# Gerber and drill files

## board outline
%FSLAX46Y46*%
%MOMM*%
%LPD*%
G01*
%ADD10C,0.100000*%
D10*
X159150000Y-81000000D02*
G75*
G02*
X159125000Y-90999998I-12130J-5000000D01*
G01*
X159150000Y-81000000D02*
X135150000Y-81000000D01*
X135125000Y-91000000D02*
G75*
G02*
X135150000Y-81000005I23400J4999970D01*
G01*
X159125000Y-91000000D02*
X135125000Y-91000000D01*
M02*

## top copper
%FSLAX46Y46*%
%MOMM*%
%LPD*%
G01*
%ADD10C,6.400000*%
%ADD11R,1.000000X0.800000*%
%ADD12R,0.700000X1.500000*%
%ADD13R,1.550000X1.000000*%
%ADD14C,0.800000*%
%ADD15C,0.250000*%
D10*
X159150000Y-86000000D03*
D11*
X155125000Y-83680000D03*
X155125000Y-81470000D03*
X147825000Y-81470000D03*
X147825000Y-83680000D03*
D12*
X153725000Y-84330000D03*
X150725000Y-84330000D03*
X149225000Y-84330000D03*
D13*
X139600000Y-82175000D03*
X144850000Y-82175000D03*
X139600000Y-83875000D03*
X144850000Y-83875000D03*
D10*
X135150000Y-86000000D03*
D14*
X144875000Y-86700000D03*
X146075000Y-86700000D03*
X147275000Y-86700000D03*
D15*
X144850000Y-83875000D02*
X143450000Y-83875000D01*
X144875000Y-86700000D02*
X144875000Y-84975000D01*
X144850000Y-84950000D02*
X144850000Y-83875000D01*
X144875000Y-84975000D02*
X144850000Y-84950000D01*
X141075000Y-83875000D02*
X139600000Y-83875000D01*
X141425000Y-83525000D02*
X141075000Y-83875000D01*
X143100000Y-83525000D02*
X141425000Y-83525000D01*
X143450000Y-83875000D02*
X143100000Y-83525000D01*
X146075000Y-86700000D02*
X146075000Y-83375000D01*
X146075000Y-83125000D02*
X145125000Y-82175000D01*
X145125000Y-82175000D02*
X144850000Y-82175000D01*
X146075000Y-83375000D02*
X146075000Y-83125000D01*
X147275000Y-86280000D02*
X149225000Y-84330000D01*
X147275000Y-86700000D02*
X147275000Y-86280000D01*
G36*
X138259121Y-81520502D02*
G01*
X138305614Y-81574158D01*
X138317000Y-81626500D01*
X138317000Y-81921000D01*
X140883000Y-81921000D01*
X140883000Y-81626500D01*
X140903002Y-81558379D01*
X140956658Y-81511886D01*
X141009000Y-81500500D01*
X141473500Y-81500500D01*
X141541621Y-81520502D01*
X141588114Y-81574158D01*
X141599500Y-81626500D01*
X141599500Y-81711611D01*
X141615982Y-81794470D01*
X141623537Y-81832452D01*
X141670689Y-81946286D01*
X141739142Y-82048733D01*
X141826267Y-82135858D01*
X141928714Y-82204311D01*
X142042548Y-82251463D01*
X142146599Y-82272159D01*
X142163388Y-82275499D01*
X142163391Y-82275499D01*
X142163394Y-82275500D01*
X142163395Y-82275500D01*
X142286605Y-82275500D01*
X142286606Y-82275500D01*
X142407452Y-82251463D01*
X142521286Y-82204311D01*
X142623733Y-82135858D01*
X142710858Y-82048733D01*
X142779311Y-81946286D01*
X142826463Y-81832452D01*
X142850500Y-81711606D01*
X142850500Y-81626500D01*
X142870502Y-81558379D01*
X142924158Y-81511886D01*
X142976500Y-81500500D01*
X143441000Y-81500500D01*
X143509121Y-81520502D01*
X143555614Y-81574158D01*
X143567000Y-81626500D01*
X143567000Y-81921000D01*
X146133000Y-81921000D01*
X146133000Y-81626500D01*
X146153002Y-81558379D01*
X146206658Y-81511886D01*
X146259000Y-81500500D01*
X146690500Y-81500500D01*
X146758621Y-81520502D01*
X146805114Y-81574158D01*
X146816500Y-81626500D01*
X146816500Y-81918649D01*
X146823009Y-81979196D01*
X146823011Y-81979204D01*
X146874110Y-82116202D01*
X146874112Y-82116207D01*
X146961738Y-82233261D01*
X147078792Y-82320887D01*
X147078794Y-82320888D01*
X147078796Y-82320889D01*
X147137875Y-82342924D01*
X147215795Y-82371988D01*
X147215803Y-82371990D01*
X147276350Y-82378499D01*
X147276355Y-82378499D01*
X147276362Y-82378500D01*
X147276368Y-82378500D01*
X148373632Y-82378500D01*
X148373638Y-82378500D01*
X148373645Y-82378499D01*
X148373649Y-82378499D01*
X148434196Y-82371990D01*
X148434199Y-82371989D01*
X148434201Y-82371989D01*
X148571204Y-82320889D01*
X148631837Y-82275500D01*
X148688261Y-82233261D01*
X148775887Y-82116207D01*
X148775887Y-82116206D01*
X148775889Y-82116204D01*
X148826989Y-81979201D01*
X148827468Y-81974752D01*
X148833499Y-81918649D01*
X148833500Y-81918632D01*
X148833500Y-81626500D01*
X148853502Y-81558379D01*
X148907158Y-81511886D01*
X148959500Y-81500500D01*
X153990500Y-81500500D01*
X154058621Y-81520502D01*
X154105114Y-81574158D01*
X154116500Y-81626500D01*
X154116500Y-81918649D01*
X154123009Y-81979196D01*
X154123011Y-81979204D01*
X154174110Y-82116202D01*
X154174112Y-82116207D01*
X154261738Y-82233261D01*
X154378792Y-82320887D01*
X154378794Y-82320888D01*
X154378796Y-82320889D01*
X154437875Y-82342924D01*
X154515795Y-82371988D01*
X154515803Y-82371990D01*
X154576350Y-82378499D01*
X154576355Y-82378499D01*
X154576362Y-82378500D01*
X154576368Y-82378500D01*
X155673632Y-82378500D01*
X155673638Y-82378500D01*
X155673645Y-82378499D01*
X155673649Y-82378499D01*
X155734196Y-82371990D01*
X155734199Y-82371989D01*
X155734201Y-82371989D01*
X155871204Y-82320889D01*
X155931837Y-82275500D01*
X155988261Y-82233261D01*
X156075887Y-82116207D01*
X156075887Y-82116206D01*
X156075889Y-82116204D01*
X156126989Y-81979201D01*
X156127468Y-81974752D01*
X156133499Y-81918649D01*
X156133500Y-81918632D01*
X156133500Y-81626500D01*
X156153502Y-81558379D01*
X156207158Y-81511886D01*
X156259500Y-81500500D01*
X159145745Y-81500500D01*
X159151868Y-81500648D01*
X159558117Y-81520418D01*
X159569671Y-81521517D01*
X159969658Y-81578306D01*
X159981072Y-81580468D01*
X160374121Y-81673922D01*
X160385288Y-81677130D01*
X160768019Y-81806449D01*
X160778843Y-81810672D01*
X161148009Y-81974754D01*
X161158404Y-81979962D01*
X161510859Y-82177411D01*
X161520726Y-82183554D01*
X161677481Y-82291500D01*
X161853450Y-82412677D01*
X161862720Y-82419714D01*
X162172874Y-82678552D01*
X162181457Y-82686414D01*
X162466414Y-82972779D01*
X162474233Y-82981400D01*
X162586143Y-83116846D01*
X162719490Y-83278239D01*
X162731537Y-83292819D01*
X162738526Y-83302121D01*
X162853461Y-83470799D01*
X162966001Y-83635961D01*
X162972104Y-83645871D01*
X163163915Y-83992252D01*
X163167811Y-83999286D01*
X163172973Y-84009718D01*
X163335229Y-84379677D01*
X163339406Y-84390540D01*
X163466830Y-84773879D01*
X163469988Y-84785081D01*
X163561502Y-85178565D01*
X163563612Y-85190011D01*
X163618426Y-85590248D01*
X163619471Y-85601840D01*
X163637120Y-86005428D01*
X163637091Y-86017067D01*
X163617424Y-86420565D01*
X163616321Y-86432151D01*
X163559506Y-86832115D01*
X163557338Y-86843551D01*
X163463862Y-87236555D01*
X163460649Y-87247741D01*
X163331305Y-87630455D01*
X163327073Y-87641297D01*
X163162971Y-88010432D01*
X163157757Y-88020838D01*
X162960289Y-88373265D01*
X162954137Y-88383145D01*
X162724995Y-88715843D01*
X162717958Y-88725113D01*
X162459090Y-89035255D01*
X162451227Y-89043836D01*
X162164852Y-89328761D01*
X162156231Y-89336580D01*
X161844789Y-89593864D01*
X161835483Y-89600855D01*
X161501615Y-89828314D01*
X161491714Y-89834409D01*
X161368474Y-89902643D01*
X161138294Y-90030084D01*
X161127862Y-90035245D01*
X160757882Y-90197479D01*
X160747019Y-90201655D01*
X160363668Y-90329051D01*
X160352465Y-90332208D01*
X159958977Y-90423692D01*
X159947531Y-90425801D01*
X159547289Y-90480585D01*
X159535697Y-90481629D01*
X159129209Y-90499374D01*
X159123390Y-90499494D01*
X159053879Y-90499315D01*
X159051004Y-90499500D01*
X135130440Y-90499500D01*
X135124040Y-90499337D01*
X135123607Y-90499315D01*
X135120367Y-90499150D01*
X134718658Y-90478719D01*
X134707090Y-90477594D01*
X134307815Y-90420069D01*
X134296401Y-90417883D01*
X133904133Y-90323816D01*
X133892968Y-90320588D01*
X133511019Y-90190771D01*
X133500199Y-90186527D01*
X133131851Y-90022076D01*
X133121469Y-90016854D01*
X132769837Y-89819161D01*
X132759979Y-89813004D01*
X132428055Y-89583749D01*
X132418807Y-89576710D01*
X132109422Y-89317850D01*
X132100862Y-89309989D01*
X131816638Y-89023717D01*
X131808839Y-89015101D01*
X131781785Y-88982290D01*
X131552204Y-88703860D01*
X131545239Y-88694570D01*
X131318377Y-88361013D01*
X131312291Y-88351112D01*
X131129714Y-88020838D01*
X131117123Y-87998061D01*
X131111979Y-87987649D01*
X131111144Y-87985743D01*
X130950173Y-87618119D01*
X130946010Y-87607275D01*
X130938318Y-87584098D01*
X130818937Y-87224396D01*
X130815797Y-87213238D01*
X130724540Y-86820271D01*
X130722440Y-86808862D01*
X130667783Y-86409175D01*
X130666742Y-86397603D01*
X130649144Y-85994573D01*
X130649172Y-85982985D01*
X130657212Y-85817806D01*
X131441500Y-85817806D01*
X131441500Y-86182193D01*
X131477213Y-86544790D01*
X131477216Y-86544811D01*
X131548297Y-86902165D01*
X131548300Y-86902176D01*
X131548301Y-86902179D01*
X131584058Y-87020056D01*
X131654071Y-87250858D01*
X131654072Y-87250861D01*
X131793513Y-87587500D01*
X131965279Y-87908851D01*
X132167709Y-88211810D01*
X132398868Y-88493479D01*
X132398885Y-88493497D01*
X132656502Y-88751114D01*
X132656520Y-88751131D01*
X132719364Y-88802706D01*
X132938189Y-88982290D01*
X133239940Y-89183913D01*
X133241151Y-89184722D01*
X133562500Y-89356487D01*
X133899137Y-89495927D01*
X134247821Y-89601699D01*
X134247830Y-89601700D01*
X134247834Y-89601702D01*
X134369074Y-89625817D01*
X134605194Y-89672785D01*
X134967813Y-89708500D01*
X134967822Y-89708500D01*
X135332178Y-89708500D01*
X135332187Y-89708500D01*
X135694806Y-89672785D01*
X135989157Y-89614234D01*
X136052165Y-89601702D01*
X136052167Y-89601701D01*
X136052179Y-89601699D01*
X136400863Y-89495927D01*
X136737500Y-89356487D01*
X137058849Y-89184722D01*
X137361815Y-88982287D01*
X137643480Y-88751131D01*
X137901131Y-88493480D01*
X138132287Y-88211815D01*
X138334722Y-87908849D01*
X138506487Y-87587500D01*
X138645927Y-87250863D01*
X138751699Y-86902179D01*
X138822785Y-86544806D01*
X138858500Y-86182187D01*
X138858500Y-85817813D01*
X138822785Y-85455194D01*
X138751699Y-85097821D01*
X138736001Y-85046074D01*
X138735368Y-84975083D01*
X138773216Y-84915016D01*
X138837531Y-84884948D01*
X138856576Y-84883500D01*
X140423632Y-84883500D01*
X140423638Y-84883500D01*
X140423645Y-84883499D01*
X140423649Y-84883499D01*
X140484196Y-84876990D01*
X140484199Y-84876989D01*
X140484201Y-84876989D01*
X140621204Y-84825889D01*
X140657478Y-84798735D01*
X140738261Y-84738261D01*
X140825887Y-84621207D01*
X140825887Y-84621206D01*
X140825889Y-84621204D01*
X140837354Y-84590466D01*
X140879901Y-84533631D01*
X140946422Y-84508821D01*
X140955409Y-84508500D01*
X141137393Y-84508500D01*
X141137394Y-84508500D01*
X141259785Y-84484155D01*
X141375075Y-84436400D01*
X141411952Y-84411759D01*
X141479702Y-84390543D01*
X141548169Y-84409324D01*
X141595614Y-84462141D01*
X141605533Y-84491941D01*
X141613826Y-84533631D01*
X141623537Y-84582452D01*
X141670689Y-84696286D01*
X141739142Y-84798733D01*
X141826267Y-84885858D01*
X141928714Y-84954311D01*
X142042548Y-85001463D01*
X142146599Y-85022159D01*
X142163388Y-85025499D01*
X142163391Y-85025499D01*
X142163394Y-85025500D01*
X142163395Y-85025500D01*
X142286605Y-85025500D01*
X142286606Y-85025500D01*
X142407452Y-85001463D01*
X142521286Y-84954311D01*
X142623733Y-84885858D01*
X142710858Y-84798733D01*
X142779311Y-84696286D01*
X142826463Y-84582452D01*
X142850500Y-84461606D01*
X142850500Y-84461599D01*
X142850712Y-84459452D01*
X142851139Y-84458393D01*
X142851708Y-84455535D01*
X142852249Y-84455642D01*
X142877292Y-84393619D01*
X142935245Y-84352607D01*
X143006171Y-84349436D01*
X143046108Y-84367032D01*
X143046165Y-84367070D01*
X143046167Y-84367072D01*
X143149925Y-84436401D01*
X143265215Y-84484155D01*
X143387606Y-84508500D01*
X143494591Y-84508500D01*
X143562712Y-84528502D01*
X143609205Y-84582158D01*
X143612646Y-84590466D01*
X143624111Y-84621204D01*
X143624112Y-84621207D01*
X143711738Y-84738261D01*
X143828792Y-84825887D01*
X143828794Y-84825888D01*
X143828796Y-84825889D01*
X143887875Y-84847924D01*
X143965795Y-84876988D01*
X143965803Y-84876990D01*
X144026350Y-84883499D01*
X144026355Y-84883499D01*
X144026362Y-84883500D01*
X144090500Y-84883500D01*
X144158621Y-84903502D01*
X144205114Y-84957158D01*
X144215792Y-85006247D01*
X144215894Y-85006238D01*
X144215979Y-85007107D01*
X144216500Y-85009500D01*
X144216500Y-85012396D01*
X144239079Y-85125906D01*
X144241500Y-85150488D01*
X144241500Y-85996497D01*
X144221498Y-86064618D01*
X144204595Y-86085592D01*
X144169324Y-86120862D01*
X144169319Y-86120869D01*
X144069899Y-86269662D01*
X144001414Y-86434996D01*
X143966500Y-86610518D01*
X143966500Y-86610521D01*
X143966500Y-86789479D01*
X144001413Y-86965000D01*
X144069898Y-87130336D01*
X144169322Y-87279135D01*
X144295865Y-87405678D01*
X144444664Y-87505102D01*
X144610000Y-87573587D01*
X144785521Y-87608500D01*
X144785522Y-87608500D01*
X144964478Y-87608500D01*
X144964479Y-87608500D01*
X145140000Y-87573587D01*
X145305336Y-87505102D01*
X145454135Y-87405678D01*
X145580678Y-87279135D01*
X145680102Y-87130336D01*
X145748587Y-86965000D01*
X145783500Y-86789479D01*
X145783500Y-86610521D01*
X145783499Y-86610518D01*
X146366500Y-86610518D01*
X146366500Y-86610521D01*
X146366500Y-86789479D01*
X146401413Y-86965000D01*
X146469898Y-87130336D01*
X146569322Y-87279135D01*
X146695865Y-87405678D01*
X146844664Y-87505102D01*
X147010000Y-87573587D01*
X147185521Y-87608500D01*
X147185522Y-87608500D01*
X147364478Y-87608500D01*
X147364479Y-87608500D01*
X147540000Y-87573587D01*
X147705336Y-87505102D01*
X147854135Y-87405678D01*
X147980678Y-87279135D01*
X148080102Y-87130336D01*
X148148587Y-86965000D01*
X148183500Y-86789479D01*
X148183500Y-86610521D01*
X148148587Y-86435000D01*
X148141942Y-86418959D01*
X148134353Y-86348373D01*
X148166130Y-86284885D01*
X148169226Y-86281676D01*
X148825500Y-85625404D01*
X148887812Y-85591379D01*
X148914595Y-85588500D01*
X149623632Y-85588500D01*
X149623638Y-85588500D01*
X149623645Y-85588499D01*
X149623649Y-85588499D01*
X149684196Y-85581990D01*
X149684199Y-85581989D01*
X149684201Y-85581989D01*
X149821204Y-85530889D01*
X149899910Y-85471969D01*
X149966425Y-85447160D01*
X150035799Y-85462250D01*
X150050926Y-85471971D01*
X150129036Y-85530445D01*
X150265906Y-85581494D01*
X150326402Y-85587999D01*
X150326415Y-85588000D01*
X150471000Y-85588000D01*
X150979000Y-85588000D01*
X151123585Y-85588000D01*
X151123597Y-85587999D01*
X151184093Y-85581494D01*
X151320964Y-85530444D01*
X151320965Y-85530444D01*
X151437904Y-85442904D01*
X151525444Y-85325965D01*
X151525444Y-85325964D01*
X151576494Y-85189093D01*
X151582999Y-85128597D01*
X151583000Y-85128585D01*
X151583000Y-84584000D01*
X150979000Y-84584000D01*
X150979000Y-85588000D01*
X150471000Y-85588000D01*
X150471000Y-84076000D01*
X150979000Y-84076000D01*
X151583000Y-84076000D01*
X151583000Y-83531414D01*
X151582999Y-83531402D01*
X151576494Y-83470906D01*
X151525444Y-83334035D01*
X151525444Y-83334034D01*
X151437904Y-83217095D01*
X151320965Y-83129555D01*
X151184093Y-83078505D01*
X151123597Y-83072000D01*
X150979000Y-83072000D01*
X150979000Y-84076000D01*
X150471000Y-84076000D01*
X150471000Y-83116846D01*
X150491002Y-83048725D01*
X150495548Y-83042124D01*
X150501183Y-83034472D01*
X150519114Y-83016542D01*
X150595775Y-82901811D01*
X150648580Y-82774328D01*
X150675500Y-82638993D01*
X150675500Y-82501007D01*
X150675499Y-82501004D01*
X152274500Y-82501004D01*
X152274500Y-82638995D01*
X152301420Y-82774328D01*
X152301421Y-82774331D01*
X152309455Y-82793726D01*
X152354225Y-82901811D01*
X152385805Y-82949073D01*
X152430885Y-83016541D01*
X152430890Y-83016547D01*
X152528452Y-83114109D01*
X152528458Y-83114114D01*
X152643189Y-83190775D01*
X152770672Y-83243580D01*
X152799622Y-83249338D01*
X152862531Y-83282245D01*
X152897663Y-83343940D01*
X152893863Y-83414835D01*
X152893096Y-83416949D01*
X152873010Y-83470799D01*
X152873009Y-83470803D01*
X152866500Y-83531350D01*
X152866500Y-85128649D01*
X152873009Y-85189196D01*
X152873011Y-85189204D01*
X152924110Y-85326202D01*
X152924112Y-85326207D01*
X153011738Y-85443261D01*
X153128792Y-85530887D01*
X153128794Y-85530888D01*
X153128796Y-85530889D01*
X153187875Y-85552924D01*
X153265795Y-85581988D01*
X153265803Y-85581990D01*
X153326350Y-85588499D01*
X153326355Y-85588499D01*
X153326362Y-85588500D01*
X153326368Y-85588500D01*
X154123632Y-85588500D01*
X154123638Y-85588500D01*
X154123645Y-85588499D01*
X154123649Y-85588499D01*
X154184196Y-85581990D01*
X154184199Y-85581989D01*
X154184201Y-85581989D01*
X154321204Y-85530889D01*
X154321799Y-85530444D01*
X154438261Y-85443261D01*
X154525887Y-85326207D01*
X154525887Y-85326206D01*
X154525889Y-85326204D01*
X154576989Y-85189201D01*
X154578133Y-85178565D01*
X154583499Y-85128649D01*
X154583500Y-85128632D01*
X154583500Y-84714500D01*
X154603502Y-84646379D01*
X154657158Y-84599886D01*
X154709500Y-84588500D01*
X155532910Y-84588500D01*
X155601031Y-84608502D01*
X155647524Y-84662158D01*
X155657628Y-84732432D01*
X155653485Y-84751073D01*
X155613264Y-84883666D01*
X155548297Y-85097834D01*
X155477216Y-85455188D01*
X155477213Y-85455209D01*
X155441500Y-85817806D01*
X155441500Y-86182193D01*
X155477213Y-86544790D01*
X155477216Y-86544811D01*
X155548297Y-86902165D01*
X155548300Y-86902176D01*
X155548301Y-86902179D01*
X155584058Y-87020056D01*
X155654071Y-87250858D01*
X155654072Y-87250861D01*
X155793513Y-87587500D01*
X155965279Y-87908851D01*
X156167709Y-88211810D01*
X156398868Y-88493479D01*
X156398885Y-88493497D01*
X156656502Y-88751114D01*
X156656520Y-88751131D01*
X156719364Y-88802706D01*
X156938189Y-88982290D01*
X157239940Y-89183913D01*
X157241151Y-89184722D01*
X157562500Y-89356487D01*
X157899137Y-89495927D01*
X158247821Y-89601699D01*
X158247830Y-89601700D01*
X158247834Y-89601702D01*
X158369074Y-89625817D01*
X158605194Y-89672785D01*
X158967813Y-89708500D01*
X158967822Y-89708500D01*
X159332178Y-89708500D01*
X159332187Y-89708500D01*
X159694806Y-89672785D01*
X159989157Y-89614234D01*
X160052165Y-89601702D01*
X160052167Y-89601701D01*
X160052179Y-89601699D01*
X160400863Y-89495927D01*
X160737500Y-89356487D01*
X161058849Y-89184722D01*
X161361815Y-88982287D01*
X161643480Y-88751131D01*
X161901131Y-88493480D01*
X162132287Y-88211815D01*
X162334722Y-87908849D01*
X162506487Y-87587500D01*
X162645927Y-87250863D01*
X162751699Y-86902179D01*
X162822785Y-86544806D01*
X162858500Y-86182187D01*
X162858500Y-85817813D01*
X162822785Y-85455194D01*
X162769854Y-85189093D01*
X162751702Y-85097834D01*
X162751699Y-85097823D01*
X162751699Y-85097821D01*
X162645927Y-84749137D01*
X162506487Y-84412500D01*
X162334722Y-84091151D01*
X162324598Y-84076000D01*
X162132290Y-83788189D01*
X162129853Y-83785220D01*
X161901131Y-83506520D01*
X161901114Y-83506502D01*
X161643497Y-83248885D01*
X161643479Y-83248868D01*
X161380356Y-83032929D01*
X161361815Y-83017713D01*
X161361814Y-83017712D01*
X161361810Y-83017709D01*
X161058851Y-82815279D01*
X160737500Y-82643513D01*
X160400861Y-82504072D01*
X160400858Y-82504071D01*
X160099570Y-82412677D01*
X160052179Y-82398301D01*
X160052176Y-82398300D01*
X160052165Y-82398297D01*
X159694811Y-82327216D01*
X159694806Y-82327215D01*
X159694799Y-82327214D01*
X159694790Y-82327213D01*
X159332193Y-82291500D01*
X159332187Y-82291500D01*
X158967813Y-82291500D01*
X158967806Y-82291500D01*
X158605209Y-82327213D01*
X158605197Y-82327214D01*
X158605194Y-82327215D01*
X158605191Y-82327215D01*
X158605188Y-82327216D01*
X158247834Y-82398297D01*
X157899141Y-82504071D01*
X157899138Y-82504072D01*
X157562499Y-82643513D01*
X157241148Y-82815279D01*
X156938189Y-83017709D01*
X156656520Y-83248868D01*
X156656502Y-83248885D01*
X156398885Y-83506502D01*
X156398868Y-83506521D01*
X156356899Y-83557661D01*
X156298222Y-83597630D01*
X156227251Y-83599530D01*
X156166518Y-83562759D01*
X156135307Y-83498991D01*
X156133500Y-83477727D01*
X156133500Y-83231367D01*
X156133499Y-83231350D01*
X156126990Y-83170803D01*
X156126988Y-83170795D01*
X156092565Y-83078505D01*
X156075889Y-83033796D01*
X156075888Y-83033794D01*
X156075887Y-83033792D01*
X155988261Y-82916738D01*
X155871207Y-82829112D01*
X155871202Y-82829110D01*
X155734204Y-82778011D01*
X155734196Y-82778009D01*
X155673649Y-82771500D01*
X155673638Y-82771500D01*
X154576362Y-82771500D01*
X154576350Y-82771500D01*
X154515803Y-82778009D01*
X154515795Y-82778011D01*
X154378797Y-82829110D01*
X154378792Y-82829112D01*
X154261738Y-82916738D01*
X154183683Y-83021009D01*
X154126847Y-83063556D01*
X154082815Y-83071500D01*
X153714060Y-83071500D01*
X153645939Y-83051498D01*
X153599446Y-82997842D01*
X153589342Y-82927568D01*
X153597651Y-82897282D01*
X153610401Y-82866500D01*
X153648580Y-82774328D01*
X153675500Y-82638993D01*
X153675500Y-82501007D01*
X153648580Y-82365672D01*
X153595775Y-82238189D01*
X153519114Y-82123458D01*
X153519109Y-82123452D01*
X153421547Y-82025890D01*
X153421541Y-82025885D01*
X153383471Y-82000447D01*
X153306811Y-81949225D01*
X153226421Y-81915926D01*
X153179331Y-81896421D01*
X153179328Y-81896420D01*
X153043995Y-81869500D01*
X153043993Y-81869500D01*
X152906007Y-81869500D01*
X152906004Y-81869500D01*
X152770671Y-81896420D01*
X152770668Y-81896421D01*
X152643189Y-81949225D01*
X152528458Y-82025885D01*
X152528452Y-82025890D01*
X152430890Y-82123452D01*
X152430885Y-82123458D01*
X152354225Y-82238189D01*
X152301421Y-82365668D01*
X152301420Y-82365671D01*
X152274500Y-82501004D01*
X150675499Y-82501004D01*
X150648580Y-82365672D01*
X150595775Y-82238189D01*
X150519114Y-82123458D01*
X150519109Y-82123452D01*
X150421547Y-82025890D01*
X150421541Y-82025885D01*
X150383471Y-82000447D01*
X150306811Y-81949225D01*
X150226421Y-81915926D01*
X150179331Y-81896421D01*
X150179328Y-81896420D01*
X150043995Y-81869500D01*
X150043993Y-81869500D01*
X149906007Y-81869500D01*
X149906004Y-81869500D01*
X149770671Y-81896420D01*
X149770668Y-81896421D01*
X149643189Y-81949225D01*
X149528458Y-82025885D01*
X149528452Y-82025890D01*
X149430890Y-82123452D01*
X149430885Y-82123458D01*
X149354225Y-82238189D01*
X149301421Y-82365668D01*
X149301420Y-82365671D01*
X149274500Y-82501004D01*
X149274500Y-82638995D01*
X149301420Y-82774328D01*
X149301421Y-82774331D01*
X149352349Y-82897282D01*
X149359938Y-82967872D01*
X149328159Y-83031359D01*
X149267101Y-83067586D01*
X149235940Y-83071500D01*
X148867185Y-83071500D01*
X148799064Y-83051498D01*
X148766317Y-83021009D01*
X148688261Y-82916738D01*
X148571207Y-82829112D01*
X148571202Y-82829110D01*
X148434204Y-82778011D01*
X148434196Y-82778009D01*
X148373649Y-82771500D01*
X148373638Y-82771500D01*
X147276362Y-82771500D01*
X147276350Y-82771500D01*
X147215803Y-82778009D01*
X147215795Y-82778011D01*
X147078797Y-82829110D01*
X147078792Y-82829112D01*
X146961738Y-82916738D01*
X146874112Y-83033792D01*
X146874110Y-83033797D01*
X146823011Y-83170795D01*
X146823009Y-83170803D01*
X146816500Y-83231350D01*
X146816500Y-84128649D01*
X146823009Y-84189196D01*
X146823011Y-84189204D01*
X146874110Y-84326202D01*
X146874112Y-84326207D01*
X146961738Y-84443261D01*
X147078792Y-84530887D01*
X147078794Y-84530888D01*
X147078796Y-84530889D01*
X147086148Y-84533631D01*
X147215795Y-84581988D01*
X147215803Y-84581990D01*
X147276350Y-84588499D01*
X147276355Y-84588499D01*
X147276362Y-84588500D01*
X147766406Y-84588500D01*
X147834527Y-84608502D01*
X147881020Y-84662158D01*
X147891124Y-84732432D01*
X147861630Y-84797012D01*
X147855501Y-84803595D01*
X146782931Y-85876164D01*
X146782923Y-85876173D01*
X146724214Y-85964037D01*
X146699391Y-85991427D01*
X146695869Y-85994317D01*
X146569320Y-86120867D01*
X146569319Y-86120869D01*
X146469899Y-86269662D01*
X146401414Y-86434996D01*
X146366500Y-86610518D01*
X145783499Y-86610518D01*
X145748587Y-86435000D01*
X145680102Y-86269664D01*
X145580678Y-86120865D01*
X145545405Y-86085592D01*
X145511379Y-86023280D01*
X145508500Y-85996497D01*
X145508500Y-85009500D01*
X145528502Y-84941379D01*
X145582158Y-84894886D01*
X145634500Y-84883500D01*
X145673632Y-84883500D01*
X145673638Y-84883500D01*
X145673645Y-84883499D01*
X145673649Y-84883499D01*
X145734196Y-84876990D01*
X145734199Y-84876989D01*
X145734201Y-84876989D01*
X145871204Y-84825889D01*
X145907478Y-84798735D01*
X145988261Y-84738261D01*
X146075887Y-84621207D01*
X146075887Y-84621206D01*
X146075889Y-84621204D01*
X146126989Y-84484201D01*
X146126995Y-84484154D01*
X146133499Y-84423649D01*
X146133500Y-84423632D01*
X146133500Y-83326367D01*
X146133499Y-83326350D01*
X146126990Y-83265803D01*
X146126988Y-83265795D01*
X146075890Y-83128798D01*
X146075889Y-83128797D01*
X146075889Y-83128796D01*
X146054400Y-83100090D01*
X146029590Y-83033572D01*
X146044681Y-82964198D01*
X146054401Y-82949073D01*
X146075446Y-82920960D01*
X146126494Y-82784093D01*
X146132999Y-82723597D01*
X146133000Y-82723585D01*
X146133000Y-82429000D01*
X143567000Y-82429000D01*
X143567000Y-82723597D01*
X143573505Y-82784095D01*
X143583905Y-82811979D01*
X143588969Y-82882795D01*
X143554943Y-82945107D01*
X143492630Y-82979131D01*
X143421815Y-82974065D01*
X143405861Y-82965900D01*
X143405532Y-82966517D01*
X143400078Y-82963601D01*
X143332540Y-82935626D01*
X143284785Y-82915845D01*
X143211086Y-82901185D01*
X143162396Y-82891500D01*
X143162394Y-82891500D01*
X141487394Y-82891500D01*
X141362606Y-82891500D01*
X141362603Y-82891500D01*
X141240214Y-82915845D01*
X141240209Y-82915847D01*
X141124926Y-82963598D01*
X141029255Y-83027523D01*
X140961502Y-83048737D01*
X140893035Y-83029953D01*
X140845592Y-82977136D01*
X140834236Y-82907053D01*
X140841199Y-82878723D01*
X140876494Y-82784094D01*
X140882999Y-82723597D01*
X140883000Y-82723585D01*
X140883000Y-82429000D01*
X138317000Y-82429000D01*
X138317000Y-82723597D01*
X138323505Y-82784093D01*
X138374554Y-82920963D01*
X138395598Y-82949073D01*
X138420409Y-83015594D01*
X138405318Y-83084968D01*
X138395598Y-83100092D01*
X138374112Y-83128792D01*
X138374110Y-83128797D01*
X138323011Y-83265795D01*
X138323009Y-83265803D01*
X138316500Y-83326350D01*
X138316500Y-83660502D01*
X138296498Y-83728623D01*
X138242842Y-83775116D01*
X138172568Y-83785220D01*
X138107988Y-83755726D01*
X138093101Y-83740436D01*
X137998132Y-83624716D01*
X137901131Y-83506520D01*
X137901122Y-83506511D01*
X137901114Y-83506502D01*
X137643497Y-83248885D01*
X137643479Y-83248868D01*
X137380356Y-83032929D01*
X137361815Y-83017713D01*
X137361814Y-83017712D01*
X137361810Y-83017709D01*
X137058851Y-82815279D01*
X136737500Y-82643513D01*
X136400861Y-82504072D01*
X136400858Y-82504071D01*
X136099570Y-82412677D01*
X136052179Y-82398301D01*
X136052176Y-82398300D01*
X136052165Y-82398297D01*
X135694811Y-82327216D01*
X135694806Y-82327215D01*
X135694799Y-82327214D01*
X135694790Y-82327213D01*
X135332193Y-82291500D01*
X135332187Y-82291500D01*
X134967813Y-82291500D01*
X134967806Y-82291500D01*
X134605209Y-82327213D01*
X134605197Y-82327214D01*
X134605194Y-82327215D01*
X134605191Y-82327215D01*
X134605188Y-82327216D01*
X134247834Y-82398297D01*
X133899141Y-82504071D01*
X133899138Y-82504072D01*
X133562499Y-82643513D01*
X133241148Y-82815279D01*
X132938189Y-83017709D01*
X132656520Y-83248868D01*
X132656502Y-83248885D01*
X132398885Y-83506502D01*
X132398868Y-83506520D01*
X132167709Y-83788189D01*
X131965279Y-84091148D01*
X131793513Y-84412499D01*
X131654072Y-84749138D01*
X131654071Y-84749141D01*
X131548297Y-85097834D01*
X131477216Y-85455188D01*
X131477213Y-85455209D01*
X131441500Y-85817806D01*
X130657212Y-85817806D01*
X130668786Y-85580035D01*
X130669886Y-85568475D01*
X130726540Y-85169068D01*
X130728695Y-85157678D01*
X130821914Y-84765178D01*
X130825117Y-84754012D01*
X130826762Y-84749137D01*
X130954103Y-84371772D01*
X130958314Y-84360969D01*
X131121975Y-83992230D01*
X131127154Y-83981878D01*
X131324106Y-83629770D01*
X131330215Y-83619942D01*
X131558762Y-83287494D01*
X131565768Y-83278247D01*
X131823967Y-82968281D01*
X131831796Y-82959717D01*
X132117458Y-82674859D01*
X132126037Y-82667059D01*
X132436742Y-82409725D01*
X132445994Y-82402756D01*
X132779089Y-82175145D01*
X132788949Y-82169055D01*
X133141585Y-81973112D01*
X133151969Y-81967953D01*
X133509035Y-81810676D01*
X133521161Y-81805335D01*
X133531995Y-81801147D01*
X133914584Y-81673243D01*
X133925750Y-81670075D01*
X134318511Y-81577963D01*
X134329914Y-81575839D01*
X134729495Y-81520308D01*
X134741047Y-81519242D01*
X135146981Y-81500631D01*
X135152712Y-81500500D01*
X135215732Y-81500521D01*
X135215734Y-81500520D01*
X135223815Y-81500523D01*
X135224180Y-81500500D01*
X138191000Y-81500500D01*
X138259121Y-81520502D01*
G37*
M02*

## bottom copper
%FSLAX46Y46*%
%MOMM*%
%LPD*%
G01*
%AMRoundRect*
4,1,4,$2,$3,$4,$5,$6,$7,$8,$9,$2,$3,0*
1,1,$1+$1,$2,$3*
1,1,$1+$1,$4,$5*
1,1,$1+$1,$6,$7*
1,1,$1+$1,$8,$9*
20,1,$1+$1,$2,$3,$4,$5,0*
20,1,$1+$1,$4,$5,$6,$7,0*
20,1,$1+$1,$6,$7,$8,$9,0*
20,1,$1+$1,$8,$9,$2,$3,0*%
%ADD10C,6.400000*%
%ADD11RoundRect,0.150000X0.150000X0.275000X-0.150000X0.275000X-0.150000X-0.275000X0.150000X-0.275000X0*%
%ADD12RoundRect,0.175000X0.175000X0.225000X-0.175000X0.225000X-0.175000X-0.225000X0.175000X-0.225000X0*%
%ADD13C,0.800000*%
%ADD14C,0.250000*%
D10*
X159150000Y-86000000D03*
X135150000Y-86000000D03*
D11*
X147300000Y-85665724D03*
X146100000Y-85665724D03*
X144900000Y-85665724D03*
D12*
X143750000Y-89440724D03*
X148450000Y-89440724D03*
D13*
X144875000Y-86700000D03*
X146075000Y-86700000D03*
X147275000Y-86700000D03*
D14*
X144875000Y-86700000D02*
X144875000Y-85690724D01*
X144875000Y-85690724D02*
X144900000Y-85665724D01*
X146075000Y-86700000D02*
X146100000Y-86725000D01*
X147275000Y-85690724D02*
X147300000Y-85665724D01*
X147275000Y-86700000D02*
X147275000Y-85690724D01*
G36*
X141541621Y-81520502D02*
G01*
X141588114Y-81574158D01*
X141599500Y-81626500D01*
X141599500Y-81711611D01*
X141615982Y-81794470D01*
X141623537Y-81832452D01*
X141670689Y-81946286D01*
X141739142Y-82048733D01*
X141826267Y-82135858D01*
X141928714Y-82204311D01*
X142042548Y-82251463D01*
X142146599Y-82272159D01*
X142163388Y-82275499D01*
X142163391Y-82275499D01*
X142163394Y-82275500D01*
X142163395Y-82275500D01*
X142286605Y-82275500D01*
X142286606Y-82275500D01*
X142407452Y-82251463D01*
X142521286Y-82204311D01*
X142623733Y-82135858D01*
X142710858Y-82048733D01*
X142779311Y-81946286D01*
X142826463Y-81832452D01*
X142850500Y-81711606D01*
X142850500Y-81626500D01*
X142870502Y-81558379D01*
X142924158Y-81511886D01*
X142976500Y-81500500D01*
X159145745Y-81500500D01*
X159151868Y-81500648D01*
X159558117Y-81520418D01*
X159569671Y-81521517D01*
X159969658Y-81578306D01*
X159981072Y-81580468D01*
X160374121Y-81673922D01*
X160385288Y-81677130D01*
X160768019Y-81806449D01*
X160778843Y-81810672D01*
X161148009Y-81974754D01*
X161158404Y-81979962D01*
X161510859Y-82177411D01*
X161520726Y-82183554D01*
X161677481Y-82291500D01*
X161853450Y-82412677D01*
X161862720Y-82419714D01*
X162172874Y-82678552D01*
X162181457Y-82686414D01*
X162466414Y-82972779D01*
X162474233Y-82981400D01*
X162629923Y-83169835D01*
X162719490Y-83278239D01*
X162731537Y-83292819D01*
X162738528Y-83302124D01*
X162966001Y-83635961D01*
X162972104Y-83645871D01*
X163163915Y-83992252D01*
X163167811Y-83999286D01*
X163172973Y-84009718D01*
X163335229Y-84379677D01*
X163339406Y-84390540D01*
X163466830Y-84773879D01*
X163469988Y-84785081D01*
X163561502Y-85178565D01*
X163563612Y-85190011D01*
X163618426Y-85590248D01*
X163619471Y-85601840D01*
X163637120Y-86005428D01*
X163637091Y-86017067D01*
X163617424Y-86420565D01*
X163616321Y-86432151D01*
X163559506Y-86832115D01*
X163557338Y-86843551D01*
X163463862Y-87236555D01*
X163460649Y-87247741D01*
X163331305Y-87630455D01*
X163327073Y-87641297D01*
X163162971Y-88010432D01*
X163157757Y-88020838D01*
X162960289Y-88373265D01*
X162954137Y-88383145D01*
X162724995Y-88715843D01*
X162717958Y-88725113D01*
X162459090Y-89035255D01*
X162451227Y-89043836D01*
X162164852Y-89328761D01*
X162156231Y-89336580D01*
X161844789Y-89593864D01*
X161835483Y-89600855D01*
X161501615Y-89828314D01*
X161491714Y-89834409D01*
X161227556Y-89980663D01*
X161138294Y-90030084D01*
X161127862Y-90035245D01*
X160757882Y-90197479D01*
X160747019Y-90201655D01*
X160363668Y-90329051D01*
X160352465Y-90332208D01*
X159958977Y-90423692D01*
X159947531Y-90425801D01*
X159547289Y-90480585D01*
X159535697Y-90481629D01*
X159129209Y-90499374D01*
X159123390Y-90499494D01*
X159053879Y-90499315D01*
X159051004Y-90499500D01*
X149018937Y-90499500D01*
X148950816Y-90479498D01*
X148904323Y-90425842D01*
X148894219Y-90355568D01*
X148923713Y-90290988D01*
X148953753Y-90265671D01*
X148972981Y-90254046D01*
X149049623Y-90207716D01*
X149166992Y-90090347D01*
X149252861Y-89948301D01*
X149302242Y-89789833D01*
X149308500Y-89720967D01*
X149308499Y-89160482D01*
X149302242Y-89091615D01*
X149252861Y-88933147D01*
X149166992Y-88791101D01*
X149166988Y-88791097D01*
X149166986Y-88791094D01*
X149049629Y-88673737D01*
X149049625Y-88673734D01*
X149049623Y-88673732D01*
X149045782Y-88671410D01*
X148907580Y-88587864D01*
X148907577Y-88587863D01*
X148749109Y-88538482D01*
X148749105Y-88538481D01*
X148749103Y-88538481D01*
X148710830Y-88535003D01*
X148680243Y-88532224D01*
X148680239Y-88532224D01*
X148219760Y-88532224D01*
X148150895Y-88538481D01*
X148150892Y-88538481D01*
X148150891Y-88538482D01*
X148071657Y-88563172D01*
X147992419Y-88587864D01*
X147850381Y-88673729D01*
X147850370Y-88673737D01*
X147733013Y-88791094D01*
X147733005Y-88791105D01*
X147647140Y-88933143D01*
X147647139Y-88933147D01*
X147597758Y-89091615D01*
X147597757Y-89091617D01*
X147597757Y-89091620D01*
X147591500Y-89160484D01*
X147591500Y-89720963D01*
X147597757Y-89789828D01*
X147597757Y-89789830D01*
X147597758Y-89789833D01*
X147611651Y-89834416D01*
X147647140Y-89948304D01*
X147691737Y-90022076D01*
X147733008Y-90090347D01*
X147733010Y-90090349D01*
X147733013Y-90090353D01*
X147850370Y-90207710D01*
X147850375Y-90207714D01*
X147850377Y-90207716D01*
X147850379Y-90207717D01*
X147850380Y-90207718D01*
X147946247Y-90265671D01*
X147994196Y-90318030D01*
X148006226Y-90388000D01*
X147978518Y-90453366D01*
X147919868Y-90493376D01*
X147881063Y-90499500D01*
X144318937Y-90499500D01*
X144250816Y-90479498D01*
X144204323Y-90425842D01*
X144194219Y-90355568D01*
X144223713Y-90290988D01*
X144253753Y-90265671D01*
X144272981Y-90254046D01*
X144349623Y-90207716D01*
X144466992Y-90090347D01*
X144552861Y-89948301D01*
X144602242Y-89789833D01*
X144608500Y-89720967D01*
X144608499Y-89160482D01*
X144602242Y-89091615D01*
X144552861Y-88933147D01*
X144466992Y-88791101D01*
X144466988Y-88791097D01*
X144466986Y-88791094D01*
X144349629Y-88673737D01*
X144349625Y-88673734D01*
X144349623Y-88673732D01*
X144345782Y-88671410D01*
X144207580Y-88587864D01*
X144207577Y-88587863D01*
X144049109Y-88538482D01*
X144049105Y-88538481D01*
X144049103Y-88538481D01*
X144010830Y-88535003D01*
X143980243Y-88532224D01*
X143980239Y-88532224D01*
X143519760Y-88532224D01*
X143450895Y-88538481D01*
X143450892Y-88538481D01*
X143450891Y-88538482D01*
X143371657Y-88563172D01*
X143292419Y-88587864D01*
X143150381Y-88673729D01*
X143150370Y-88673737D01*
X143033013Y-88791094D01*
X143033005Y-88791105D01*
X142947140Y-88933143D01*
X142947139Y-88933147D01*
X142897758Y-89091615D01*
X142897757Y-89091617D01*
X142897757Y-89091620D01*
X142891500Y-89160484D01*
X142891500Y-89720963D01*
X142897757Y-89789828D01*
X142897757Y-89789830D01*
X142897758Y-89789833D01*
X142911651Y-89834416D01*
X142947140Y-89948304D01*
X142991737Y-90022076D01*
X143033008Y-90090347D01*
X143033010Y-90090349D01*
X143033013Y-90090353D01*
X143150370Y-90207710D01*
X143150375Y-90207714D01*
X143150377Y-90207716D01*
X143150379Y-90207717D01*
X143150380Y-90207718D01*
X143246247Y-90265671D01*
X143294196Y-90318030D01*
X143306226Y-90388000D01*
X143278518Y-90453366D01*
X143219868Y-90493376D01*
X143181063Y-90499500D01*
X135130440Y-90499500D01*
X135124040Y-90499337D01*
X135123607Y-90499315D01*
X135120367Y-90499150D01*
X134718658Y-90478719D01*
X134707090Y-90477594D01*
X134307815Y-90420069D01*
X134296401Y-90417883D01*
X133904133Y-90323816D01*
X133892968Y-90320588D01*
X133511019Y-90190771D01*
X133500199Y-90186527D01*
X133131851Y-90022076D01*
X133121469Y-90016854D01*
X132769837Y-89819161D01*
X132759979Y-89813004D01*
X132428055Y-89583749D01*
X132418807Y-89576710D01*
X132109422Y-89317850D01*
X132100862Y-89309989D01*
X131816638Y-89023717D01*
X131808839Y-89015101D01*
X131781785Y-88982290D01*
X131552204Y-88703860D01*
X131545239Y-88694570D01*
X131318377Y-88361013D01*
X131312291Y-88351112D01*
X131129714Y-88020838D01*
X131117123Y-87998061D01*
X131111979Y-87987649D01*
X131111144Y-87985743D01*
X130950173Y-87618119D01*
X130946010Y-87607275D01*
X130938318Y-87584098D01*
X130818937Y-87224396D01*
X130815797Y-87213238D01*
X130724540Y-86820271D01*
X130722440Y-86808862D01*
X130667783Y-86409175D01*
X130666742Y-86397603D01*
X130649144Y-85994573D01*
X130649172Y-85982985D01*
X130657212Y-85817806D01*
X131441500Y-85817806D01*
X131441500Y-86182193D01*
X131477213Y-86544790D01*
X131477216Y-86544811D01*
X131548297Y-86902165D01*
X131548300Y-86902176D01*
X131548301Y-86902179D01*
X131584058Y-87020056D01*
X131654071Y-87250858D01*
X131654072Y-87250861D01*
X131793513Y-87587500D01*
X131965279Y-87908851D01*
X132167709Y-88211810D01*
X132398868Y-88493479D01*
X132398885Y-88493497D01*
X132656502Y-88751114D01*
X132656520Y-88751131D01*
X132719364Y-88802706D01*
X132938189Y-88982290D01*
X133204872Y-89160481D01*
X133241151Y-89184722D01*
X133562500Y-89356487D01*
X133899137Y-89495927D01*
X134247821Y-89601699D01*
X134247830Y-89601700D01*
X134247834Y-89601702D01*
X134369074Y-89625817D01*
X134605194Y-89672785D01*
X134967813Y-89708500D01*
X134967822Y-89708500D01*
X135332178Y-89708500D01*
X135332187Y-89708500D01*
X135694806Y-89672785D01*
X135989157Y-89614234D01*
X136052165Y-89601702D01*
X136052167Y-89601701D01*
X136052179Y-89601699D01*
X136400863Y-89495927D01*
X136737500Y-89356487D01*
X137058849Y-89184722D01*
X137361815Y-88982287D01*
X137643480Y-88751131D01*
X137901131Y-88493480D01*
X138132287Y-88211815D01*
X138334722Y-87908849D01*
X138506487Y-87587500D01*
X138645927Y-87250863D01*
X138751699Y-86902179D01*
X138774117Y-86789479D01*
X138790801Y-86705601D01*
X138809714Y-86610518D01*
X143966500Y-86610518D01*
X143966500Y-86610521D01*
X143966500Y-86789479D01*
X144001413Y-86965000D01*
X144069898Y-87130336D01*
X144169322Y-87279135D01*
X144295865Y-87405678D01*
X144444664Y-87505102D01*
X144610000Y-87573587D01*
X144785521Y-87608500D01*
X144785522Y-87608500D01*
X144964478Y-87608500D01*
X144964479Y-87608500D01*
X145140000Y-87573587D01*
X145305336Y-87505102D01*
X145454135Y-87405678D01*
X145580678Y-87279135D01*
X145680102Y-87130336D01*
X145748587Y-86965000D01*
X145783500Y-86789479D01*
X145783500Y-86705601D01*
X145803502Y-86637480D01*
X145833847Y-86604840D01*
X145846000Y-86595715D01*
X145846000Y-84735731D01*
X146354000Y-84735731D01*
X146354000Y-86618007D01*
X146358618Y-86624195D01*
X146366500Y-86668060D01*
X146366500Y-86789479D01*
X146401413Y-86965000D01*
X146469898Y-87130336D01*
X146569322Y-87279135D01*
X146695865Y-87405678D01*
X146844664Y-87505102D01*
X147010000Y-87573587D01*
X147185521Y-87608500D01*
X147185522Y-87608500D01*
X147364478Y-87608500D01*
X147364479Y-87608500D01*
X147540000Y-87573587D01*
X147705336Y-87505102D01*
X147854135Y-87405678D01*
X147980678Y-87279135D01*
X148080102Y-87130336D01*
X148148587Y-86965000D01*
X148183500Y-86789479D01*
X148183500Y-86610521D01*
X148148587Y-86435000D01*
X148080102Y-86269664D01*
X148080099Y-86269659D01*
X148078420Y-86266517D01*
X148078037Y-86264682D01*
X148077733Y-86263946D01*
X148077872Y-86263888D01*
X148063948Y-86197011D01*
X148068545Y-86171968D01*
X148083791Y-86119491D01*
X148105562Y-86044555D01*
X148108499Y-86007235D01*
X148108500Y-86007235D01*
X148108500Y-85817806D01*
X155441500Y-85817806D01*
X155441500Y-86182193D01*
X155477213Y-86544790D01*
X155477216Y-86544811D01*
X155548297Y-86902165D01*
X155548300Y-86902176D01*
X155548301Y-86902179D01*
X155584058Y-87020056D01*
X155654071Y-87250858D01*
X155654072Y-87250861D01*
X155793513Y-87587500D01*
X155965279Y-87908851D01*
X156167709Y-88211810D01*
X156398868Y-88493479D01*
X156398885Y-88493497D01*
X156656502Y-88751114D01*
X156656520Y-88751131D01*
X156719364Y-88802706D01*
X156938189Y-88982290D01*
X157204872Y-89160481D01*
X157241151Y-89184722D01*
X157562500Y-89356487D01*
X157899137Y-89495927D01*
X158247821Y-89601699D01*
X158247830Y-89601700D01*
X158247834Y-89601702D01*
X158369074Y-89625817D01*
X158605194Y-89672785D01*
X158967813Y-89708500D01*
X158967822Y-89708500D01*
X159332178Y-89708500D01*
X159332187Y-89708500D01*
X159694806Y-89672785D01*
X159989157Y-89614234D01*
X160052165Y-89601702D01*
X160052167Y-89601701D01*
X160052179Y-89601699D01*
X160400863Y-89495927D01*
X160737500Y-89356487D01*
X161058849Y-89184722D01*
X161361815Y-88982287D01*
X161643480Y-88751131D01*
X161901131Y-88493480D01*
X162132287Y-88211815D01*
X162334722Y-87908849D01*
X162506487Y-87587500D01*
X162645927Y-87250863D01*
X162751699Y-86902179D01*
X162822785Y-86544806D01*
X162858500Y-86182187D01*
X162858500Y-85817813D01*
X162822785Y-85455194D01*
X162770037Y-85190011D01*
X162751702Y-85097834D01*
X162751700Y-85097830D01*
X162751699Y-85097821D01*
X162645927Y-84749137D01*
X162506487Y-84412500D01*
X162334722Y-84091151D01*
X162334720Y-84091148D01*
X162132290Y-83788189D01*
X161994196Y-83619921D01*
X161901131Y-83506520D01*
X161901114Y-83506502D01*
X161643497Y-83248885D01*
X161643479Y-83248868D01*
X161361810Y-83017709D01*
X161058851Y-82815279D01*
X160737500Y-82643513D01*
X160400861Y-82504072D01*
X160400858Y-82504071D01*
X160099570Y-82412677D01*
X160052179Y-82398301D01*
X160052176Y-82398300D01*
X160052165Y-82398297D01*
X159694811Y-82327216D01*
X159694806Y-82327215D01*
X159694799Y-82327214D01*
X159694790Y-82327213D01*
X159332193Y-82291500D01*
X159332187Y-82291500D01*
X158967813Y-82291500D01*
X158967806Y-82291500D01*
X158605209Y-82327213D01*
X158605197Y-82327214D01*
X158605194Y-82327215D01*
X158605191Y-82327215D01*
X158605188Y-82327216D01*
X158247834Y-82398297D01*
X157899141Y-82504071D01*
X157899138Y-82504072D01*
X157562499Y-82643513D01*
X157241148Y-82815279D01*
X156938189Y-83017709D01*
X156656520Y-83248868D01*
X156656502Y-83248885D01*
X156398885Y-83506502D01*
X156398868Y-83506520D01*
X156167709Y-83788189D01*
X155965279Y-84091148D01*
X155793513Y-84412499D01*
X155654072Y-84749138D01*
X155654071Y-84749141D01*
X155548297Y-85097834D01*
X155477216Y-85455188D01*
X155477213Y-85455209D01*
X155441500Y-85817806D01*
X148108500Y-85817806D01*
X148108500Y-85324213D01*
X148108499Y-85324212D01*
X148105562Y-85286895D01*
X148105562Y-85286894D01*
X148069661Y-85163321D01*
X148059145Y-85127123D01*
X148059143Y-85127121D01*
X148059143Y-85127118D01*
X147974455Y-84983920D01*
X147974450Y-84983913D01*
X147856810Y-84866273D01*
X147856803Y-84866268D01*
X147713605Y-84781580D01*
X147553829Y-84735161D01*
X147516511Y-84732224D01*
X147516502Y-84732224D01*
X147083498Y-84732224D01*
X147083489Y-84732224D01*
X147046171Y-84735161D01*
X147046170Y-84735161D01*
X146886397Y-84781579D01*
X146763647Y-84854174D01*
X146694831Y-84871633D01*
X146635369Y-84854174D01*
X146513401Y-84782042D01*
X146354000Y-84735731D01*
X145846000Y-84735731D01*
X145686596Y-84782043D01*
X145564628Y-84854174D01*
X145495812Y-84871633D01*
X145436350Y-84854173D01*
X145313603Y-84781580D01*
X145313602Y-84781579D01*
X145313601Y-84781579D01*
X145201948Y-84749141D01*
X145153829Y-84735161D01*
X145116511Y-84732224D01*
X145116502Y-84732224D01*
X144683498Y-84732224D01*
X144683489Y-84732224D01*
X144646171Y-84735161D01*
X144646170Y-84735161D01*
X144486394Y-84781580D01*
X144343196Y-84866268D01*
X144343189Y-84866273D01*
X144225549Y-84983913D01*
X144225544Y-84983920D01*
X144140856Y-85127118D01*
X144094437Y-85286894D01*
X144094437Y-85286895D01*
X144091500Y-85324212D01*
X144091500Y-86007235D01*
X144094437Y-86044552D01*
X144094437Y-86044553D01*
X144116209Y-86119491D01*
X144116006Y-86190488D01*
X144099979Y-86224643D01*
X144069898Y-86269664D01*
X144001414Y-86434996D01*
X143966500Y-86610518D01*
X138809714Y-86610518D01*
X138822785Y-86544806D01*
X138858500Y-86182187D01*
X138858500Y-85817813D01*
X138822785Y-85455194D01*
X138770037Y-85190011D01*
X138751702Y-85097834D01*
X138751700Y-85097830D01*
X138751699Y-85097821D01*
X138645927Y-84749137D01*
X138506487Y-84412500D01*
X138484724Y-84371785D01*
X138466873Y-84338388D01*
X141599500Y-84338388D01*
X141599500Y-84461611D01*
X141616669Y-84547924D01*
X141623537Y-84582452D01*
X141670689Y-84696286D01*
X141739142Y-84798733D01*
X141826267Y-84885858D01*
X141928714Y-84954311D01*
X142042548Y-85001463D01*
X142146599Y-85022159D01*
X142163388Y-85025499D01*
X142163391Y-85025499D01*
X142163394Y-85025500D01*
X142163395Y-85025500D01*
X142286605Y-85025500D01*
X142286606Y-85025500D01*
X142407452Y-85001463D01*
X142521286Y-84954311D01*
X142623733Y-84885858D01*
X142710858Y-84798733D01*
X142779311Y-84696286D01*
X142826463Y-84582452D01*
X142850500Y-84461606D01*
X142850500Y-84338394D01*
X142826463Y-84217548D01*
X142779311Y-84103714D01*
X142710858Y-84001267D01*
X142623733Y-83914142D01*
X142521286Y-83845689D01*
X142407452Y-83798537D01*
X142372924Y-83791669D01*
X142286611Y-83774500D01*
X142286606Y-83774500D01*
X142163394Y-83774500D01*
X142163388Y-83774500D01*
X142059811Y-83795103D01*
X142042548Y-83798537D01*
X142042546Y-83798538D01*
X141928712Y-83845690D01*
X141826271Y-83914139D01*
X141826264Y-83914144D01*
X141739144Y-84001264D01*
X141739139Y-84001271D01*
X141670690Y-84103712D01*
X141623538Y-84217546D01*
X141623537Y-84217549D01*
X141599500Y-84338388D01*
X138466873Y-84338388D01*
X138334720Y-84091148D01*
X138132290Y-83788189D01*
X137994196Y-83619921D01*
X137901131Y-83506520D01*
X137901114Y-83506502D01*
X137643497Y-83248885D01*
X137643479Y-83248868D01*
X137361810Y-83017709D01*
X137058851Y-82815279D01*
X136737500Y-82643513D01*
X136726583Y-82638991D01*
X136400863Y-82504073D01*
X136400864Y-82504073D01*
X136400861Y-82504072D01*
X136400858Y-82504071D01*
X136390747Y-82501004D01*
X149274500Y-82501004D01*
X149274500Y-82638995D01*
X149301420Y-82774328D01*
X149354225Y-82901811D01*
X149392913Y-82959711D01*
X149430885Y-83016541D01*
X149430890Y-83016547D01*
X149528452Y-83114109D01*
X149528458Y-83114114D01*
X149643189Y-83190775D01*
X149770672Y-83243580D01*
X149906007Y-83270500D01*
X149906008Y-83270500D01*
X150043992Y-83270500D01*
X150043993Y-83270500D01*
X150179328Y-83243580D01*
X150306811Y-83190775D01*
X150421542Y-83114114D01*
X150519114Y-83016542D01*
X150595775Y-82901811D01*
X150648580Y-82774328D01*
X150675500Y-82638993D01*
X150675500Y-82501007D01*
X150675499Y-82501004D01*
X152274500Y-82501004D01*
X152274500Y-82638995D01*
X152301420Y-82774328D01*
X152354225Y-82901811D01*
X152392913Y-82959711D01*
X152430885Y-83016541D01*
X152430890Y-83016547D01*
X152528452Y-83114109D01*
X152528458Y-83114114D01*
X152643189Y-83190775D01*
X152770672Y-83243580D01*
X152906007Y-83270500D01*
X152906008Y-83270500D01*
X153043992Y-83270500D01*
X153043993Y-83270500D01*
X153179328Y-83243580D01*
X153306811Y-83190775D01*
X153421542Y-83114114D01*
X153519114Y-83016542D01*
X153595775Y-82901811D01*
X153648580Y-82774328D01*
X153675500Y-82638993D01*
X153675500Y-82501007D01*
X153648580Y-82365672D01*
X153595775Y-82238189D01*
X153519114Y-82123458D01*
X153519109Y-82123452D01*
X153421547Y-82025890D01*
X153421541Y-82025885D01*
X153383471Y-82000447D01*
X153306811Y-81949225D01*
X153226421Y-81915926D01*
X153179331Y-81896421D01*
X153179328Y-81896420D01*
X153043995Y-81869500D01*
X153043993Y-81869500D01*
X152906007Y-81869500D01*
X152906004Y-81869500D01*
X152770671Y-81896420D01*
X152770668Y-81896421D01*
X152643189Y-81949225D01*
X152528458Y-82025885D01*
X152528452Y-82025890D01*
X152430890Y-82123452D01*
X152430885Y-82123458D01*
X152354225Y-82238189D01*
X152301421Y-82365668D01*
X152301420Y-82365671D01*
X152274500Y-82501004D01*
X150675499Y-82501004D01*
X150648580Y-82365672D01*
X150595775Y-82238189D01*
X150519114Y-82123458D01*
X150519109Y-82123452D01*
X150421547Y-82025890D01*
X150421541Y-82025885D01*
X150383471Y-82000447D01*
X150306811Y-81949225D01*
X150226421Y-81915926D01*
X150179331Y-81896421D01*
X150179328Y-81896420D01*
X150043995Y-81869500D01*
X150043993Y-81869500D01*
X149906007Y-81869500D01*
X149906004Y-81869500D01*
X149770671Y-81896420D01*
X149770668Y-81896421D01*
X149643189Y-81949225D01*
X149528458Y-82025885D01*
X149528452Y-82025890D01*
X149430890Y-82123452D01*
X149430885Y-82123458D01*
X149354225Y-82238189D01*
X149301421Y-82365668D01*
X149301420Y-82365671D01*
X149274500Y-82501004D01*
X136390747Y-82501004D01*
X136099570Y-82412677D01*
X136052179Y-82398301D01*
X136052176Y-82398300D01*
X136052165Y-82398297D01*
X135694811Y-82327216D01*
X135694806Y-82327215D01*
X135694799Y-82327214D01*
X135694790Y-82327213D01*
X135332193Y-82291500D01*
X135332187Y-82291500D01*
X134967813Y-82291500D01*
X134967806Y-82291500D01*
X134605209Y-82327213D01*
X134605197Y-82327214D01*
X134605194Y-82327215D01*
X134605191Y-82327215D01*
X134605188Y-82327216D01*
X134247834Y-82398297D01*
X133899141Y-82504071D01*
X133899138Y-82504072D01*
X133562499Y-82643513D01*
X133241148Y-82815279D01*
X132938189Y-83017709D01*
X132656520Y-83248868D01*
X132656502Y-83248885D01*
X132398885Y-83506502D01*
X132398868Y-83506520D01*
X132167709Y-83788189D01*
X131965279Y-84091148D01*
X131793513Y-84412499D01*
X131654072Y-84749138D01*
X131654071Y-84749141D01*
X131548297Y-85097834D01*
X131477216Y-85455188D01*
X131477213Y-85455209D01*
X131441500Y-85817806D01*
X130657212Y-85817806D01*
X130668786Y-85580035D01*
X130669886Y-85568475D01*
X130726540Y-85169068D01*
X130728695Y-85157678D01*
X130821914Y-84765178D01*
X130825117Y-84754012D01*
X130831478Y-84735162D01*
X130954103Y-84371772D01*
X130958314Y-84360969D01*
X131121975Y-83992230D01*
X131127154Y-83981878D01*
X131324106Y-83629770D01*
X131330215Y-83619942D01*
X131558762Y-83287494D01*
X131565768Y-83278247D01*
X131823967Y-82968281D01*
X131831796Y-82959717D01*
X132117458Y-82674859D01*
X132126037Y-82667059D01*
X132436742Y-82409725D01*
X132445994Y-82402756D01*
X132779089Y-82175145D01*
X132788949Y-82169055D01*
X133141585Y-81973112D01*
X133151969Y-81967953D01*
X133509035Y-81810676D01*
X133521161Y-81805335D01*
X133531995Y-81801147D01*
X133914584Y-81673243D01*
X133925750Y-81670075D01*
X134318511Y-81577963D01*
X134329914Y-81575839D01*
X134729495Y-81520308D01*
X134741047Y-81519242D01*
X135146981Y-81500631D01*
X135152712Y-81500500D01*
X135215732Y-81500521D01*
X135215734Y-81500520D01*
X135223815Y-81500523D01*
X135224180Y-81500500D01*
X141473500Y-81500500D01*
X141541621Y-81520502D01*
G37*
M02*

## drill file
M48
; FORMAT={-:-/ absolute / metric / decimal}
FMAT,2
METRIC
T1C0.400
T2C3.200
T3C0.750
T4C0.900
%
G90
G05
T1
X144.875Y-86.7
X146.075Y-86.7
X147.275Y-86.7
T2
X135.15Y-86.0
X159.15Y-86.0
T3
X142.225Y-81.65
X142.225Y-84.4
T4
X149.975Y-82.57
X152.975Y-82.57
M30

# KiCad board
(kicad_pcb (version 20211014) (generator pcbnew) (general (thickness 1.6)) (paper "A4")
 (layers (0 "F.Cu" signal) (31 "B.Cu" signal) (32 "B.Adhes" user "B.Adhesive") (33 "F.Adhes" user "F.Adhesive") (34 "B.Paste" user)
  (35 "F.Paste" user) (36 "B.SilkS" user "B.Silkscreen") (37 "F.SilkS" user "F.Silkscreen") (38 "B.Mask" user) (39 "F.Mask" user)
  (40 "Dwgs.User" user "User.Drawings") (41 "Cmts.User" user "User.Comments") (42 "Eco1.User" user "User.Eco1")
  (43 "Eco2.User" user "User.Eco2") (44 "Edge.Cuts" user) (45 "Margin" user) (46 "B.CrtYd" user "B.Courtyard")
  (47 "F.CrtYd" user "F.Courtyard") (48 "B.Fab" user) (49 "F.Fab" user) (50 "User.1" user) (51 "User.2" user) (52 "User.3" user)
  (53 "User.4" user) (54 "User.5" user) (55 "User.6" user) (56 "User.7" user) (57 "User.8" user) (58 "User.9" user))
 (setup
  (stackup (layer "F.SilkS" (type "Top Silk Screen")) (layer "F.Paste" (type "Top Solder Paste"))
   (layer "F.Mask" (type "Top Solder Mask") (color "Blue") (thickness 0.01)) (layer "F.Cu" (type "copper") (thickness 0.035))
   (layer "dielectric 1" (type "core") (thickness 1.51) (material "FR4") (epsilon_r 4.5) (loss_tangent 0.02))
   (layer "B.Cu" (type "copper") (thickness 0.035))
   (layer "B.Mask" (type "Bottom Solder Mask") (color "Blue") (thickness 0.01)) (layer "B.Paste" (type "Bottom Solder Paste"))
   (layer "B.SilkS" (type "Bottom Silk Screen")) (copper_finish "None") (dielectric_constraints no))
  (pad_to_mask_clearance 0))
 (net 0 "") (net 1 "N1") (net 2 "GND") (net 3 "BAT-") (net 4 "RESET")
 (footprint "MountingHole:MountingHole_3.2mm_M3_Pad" (layer "F.Cu") (at 159.15 86)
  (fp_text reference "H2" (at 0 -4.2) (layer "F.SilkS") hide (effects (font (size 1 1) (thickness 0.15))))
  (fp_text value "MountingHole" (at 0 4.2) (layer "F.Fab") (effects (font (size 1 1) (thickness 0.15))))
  (pad "1" thru_hole circle (at 0 0) (size 6.4 6.4) (drill 3.2) (layers *.Cu *.Mask)))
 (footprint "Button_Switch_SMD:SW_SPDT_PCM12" (layer "F.Cu") (at 151.475 82.9 180)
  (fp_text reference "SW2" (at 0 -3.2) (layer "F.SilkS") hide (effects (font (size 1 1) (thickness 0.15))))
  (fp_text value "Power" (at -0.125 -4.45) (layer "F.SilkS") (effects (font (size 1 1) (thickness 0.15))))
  (pad "" smd rect (at -3.65 -0.78 180) (size 1 0.8) (layers "F.Cu" "F.Paste" "F.Mask"))
  (pad "" smd rect (at -3.65 1.43 180) (size 1 0.8) (layers "F.Cu" "F.Paste" "F.Mask"))
  (pad "" np_thru_hole circle (at -1.5 0.33 180) (size 0.9 0.9) (drill 0.9) (layers *.Cu *.Mask))
  (pad "" smd rect (at 3.65 1.43 180) (size 1 0.8) (layers "F.Cu" "F.Paste" "F.Mask"))
  (pad "" smd rect (at 3.65 -0.78 180) (size 1 0.8) (layers "F.Cu" "F.Paste" "F.Mask"))
  (pad "" np_thru_hole circle (at 1.5 0.33 180) (size 0.9 0.9) (drill 0.9) (layers *.Cu *.Mask))
  (pad "1" smd rect (at -2.25 -1.43 180) (size 0.7 1.5) (layers "F.Cu" "F.Paste" "F.Mask") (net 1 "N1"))
  (pad "2" smd rect (at 0.75 -1.43 180) (size 0.7 1.5) (layers "F.Cu" "F.Paste" "F.Mask") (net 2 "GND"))
  (pad "3" smd rect (at 2.25 -1.43 180) (size 0.7 1.5) (layers "F.Cu" "F.Paste" "F.Mask") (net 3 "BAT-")))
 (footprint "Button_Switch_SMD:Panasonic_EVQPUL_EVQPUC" (layer "F.Cu") (at 142.225 83.025)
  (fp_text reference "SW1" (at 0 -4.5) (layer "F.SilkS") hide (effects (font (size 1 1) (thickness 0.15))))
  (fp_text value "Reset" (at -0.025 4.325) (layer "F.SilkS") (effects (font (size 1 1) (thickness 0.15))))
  (pad "" np_thru_hole circle (at 0 1.375 180) (size 0.75 0.75) (drill 0.75) (layers *.Cu *.Mask))
  (pad "" np_thru_hole circle (at 0 -1.375 180) (size 0.75 0.75) (drill 0.75) (layers *.Cu *.Mask))
  (pad "1" smd rect (at -2.625 -0.85 180) (size 1.55 1) (layers "F.Cu" "F.Paste" "F.Mask") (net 2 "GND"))
  (pad "1" smd rect (at 2.625 -0.85 180) (size 1.55 1) (layers "F.Cu" "F.Paste" "F.Mask") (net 2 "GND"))
  (pad "2" smd rect (at -2.625 0.85 180) (size 1.55 1) (layers "F.Cu" "F.Paste" "F.Mask") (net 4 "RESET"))
  (pad "2" smd rect (at 2.625 0.85 180) (size 1.55 1) (layers "F.Cu" "F.Paste" "F.Mask") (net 4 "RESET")))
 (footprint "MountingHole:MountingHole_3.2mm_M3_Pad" (layer "F.Cu") (at 135.15 86)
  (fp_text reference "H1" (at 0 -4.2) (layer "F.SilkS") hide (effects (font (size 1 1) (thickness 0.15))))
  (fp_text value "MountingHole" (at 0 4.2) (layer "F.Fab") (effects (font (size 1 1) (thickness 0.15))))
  (pad "1" thru_hole circle (at 0 0) (size 6.4 6.4) (drill 3.2) (layers *.Cu *.Mask)))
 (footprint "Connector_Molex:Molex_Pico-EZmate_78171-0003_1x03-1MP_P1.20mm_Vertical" (layer "B.Cu") (at 146.1 87.540724 180)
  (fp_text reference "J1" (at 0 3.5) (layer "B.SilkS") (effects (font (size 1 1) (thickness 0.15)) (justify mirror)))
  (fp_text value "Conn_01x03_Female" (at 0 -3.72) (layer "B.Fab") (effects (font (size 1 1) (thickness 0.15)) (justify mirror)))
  (pad "1" smd roundrect (at -1.2 1.875 180) (size 0.6 0.85) (layers "B.Cu" "B.Paste" "B.Mask") (roundrect_rratio 0.25) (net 3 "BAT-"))
  (pad "2" smd roundrect (at 0 1.875 180) (size 0.6 0.85) (layers "B.Cu" "B.Paste" "B.Mask") (roundrect_rratio 0.25) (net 2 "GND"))
  (pad "3" smd roundrect (at 1.2 1.875 180) (size 0.6 0.85) (layers "B.Cu" "B.Paste" "B.Mask") (roundrect_rratio 0.25) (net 4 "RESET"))
  (pad "MP" smd roundrect (at 2.35 -1.9 180) (size 0.7 0.8) (layers "B.Cu" "B.Paste" "B.Mask") (roundrect_rratio 0.25))
  (pad "MP" smd roundrect (at -2.35 -1.9 180) (size 0.7 0.8) (layers "B.Cu" "B.Paste" "B.Mask") (roundrect_rratio 0.25)))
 (gr_arc (start 159.15 81) (mid 164.137873 86.0125) (end 159.125 91) (layer "Edge.Cuts") (width 0.1))
 (gr_line (start 159.15 81) (end 135.15 81) (layer "Edge.Cuts") (width 0.1))
 (gr_arc (start 135.125 91) (mid 130.148393 85.987527) (end 135.15 81) (layer "Edge.Cuts") (width 0.1))
 (gr_line (start 159.125 91) (end 135.125 91) (layer "Edge.Cuts") (width 0.1))
 (segment (start 144.85 83.875) (end 143.45 83.875) (width 0.25) (layer "F.Cu") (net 4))
 (segment (start 144.875 86.7) (end 144.875 84.975) (width 0.25) (layer "F.Cu") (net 4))
 (segment (start 144.85 84.95) (end 144.85 83.875) (width 0.25) (layer "F.Cu") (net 4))
 (segment (start 144.875 84.975) (end 144.85 84.95) (width 0.25) (layer "F.Cu") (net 4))
 (segment (start 141.075 83.875) (end 139.6 83.875) (width 0.25) (layer "F.Cu") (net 4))
 (segment (start 141.425 83.525) (end 141.075 83.875) (width 0.25) (layer "F.Cu") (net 4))
 (segment (start 143.1 83.525) (end 141.425 83.525) (width 0.25) (layer "F.Cu") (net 4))
 (segment (start 143.45 83.875) (end 143.1 83.525) (width 0.25) (layer "F.Cu") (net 4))
 (via (at 144.875 86.7) (size 0.8) (drill 0.4) (layers "F.Cu" "B.Cu") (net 4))
 (segment (start 144.875 86.7) (end 144.875 85.690724) (width 0.25) (layer "B.Cu") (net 4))
 (segment (start 144.875 85.690724) (end 144.9 85.665724) (width 0.25) (layer "B.Cu") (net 4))
 (segment (start 146.075 86.7) (end 146.075 83.375) (width 0.25) (layer "F.Cu") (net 2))
 (segment (start 146.075 83.125) (end 145.125 82.175) (width 0.25) (layer "F.Cu") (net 2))
 (segment (start 145.125 82.175) (end 144.85 82.175) (width 0.25) (layer "F.Cu") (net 2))
 (segment (start 146.075 83.375) (end 146.075 83.125) (width 0.25) (layer "F.Cu") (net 2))
 (via (at 146.075 86.7) (size 0.8) (drill 0.4) (layers "F.Cu" "B.Cu") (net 2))
 (segment (start 146.075 86.7) (end 146.1 86.725) (width 0.25) (layer "B.Cu") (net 2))
 (segment (start 147.275 86.28) (end 149.225 84.33) (width 0.25) (layer "F.Cu") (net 3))
 (segment (start 147.275 86.7) (end 147.275 86.28) (width 0.25) (layer "F.Cu") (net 3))
 (via (at 147.275 86.7) (size 0.8) (drill 0.4) (layers "F.Cu" "B.Cu") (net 3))
 (segment (start 147.275 85.690724) (end 147.3 85.665724) (width 0.25) (layer "B.Cu") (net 3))
 (segment (start 147.275 86.7) (end 147.275 85.690724) (width 0.25) (layer "B.Cu") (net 3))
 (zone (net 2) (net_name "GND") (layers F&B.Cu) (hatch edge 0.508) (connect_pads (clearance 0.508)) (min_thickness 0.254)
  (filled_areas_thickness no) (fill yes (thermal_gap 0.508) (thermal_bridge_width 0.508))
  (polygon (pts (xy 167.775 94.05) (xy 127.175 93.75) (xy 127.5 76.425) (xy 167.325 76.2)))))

